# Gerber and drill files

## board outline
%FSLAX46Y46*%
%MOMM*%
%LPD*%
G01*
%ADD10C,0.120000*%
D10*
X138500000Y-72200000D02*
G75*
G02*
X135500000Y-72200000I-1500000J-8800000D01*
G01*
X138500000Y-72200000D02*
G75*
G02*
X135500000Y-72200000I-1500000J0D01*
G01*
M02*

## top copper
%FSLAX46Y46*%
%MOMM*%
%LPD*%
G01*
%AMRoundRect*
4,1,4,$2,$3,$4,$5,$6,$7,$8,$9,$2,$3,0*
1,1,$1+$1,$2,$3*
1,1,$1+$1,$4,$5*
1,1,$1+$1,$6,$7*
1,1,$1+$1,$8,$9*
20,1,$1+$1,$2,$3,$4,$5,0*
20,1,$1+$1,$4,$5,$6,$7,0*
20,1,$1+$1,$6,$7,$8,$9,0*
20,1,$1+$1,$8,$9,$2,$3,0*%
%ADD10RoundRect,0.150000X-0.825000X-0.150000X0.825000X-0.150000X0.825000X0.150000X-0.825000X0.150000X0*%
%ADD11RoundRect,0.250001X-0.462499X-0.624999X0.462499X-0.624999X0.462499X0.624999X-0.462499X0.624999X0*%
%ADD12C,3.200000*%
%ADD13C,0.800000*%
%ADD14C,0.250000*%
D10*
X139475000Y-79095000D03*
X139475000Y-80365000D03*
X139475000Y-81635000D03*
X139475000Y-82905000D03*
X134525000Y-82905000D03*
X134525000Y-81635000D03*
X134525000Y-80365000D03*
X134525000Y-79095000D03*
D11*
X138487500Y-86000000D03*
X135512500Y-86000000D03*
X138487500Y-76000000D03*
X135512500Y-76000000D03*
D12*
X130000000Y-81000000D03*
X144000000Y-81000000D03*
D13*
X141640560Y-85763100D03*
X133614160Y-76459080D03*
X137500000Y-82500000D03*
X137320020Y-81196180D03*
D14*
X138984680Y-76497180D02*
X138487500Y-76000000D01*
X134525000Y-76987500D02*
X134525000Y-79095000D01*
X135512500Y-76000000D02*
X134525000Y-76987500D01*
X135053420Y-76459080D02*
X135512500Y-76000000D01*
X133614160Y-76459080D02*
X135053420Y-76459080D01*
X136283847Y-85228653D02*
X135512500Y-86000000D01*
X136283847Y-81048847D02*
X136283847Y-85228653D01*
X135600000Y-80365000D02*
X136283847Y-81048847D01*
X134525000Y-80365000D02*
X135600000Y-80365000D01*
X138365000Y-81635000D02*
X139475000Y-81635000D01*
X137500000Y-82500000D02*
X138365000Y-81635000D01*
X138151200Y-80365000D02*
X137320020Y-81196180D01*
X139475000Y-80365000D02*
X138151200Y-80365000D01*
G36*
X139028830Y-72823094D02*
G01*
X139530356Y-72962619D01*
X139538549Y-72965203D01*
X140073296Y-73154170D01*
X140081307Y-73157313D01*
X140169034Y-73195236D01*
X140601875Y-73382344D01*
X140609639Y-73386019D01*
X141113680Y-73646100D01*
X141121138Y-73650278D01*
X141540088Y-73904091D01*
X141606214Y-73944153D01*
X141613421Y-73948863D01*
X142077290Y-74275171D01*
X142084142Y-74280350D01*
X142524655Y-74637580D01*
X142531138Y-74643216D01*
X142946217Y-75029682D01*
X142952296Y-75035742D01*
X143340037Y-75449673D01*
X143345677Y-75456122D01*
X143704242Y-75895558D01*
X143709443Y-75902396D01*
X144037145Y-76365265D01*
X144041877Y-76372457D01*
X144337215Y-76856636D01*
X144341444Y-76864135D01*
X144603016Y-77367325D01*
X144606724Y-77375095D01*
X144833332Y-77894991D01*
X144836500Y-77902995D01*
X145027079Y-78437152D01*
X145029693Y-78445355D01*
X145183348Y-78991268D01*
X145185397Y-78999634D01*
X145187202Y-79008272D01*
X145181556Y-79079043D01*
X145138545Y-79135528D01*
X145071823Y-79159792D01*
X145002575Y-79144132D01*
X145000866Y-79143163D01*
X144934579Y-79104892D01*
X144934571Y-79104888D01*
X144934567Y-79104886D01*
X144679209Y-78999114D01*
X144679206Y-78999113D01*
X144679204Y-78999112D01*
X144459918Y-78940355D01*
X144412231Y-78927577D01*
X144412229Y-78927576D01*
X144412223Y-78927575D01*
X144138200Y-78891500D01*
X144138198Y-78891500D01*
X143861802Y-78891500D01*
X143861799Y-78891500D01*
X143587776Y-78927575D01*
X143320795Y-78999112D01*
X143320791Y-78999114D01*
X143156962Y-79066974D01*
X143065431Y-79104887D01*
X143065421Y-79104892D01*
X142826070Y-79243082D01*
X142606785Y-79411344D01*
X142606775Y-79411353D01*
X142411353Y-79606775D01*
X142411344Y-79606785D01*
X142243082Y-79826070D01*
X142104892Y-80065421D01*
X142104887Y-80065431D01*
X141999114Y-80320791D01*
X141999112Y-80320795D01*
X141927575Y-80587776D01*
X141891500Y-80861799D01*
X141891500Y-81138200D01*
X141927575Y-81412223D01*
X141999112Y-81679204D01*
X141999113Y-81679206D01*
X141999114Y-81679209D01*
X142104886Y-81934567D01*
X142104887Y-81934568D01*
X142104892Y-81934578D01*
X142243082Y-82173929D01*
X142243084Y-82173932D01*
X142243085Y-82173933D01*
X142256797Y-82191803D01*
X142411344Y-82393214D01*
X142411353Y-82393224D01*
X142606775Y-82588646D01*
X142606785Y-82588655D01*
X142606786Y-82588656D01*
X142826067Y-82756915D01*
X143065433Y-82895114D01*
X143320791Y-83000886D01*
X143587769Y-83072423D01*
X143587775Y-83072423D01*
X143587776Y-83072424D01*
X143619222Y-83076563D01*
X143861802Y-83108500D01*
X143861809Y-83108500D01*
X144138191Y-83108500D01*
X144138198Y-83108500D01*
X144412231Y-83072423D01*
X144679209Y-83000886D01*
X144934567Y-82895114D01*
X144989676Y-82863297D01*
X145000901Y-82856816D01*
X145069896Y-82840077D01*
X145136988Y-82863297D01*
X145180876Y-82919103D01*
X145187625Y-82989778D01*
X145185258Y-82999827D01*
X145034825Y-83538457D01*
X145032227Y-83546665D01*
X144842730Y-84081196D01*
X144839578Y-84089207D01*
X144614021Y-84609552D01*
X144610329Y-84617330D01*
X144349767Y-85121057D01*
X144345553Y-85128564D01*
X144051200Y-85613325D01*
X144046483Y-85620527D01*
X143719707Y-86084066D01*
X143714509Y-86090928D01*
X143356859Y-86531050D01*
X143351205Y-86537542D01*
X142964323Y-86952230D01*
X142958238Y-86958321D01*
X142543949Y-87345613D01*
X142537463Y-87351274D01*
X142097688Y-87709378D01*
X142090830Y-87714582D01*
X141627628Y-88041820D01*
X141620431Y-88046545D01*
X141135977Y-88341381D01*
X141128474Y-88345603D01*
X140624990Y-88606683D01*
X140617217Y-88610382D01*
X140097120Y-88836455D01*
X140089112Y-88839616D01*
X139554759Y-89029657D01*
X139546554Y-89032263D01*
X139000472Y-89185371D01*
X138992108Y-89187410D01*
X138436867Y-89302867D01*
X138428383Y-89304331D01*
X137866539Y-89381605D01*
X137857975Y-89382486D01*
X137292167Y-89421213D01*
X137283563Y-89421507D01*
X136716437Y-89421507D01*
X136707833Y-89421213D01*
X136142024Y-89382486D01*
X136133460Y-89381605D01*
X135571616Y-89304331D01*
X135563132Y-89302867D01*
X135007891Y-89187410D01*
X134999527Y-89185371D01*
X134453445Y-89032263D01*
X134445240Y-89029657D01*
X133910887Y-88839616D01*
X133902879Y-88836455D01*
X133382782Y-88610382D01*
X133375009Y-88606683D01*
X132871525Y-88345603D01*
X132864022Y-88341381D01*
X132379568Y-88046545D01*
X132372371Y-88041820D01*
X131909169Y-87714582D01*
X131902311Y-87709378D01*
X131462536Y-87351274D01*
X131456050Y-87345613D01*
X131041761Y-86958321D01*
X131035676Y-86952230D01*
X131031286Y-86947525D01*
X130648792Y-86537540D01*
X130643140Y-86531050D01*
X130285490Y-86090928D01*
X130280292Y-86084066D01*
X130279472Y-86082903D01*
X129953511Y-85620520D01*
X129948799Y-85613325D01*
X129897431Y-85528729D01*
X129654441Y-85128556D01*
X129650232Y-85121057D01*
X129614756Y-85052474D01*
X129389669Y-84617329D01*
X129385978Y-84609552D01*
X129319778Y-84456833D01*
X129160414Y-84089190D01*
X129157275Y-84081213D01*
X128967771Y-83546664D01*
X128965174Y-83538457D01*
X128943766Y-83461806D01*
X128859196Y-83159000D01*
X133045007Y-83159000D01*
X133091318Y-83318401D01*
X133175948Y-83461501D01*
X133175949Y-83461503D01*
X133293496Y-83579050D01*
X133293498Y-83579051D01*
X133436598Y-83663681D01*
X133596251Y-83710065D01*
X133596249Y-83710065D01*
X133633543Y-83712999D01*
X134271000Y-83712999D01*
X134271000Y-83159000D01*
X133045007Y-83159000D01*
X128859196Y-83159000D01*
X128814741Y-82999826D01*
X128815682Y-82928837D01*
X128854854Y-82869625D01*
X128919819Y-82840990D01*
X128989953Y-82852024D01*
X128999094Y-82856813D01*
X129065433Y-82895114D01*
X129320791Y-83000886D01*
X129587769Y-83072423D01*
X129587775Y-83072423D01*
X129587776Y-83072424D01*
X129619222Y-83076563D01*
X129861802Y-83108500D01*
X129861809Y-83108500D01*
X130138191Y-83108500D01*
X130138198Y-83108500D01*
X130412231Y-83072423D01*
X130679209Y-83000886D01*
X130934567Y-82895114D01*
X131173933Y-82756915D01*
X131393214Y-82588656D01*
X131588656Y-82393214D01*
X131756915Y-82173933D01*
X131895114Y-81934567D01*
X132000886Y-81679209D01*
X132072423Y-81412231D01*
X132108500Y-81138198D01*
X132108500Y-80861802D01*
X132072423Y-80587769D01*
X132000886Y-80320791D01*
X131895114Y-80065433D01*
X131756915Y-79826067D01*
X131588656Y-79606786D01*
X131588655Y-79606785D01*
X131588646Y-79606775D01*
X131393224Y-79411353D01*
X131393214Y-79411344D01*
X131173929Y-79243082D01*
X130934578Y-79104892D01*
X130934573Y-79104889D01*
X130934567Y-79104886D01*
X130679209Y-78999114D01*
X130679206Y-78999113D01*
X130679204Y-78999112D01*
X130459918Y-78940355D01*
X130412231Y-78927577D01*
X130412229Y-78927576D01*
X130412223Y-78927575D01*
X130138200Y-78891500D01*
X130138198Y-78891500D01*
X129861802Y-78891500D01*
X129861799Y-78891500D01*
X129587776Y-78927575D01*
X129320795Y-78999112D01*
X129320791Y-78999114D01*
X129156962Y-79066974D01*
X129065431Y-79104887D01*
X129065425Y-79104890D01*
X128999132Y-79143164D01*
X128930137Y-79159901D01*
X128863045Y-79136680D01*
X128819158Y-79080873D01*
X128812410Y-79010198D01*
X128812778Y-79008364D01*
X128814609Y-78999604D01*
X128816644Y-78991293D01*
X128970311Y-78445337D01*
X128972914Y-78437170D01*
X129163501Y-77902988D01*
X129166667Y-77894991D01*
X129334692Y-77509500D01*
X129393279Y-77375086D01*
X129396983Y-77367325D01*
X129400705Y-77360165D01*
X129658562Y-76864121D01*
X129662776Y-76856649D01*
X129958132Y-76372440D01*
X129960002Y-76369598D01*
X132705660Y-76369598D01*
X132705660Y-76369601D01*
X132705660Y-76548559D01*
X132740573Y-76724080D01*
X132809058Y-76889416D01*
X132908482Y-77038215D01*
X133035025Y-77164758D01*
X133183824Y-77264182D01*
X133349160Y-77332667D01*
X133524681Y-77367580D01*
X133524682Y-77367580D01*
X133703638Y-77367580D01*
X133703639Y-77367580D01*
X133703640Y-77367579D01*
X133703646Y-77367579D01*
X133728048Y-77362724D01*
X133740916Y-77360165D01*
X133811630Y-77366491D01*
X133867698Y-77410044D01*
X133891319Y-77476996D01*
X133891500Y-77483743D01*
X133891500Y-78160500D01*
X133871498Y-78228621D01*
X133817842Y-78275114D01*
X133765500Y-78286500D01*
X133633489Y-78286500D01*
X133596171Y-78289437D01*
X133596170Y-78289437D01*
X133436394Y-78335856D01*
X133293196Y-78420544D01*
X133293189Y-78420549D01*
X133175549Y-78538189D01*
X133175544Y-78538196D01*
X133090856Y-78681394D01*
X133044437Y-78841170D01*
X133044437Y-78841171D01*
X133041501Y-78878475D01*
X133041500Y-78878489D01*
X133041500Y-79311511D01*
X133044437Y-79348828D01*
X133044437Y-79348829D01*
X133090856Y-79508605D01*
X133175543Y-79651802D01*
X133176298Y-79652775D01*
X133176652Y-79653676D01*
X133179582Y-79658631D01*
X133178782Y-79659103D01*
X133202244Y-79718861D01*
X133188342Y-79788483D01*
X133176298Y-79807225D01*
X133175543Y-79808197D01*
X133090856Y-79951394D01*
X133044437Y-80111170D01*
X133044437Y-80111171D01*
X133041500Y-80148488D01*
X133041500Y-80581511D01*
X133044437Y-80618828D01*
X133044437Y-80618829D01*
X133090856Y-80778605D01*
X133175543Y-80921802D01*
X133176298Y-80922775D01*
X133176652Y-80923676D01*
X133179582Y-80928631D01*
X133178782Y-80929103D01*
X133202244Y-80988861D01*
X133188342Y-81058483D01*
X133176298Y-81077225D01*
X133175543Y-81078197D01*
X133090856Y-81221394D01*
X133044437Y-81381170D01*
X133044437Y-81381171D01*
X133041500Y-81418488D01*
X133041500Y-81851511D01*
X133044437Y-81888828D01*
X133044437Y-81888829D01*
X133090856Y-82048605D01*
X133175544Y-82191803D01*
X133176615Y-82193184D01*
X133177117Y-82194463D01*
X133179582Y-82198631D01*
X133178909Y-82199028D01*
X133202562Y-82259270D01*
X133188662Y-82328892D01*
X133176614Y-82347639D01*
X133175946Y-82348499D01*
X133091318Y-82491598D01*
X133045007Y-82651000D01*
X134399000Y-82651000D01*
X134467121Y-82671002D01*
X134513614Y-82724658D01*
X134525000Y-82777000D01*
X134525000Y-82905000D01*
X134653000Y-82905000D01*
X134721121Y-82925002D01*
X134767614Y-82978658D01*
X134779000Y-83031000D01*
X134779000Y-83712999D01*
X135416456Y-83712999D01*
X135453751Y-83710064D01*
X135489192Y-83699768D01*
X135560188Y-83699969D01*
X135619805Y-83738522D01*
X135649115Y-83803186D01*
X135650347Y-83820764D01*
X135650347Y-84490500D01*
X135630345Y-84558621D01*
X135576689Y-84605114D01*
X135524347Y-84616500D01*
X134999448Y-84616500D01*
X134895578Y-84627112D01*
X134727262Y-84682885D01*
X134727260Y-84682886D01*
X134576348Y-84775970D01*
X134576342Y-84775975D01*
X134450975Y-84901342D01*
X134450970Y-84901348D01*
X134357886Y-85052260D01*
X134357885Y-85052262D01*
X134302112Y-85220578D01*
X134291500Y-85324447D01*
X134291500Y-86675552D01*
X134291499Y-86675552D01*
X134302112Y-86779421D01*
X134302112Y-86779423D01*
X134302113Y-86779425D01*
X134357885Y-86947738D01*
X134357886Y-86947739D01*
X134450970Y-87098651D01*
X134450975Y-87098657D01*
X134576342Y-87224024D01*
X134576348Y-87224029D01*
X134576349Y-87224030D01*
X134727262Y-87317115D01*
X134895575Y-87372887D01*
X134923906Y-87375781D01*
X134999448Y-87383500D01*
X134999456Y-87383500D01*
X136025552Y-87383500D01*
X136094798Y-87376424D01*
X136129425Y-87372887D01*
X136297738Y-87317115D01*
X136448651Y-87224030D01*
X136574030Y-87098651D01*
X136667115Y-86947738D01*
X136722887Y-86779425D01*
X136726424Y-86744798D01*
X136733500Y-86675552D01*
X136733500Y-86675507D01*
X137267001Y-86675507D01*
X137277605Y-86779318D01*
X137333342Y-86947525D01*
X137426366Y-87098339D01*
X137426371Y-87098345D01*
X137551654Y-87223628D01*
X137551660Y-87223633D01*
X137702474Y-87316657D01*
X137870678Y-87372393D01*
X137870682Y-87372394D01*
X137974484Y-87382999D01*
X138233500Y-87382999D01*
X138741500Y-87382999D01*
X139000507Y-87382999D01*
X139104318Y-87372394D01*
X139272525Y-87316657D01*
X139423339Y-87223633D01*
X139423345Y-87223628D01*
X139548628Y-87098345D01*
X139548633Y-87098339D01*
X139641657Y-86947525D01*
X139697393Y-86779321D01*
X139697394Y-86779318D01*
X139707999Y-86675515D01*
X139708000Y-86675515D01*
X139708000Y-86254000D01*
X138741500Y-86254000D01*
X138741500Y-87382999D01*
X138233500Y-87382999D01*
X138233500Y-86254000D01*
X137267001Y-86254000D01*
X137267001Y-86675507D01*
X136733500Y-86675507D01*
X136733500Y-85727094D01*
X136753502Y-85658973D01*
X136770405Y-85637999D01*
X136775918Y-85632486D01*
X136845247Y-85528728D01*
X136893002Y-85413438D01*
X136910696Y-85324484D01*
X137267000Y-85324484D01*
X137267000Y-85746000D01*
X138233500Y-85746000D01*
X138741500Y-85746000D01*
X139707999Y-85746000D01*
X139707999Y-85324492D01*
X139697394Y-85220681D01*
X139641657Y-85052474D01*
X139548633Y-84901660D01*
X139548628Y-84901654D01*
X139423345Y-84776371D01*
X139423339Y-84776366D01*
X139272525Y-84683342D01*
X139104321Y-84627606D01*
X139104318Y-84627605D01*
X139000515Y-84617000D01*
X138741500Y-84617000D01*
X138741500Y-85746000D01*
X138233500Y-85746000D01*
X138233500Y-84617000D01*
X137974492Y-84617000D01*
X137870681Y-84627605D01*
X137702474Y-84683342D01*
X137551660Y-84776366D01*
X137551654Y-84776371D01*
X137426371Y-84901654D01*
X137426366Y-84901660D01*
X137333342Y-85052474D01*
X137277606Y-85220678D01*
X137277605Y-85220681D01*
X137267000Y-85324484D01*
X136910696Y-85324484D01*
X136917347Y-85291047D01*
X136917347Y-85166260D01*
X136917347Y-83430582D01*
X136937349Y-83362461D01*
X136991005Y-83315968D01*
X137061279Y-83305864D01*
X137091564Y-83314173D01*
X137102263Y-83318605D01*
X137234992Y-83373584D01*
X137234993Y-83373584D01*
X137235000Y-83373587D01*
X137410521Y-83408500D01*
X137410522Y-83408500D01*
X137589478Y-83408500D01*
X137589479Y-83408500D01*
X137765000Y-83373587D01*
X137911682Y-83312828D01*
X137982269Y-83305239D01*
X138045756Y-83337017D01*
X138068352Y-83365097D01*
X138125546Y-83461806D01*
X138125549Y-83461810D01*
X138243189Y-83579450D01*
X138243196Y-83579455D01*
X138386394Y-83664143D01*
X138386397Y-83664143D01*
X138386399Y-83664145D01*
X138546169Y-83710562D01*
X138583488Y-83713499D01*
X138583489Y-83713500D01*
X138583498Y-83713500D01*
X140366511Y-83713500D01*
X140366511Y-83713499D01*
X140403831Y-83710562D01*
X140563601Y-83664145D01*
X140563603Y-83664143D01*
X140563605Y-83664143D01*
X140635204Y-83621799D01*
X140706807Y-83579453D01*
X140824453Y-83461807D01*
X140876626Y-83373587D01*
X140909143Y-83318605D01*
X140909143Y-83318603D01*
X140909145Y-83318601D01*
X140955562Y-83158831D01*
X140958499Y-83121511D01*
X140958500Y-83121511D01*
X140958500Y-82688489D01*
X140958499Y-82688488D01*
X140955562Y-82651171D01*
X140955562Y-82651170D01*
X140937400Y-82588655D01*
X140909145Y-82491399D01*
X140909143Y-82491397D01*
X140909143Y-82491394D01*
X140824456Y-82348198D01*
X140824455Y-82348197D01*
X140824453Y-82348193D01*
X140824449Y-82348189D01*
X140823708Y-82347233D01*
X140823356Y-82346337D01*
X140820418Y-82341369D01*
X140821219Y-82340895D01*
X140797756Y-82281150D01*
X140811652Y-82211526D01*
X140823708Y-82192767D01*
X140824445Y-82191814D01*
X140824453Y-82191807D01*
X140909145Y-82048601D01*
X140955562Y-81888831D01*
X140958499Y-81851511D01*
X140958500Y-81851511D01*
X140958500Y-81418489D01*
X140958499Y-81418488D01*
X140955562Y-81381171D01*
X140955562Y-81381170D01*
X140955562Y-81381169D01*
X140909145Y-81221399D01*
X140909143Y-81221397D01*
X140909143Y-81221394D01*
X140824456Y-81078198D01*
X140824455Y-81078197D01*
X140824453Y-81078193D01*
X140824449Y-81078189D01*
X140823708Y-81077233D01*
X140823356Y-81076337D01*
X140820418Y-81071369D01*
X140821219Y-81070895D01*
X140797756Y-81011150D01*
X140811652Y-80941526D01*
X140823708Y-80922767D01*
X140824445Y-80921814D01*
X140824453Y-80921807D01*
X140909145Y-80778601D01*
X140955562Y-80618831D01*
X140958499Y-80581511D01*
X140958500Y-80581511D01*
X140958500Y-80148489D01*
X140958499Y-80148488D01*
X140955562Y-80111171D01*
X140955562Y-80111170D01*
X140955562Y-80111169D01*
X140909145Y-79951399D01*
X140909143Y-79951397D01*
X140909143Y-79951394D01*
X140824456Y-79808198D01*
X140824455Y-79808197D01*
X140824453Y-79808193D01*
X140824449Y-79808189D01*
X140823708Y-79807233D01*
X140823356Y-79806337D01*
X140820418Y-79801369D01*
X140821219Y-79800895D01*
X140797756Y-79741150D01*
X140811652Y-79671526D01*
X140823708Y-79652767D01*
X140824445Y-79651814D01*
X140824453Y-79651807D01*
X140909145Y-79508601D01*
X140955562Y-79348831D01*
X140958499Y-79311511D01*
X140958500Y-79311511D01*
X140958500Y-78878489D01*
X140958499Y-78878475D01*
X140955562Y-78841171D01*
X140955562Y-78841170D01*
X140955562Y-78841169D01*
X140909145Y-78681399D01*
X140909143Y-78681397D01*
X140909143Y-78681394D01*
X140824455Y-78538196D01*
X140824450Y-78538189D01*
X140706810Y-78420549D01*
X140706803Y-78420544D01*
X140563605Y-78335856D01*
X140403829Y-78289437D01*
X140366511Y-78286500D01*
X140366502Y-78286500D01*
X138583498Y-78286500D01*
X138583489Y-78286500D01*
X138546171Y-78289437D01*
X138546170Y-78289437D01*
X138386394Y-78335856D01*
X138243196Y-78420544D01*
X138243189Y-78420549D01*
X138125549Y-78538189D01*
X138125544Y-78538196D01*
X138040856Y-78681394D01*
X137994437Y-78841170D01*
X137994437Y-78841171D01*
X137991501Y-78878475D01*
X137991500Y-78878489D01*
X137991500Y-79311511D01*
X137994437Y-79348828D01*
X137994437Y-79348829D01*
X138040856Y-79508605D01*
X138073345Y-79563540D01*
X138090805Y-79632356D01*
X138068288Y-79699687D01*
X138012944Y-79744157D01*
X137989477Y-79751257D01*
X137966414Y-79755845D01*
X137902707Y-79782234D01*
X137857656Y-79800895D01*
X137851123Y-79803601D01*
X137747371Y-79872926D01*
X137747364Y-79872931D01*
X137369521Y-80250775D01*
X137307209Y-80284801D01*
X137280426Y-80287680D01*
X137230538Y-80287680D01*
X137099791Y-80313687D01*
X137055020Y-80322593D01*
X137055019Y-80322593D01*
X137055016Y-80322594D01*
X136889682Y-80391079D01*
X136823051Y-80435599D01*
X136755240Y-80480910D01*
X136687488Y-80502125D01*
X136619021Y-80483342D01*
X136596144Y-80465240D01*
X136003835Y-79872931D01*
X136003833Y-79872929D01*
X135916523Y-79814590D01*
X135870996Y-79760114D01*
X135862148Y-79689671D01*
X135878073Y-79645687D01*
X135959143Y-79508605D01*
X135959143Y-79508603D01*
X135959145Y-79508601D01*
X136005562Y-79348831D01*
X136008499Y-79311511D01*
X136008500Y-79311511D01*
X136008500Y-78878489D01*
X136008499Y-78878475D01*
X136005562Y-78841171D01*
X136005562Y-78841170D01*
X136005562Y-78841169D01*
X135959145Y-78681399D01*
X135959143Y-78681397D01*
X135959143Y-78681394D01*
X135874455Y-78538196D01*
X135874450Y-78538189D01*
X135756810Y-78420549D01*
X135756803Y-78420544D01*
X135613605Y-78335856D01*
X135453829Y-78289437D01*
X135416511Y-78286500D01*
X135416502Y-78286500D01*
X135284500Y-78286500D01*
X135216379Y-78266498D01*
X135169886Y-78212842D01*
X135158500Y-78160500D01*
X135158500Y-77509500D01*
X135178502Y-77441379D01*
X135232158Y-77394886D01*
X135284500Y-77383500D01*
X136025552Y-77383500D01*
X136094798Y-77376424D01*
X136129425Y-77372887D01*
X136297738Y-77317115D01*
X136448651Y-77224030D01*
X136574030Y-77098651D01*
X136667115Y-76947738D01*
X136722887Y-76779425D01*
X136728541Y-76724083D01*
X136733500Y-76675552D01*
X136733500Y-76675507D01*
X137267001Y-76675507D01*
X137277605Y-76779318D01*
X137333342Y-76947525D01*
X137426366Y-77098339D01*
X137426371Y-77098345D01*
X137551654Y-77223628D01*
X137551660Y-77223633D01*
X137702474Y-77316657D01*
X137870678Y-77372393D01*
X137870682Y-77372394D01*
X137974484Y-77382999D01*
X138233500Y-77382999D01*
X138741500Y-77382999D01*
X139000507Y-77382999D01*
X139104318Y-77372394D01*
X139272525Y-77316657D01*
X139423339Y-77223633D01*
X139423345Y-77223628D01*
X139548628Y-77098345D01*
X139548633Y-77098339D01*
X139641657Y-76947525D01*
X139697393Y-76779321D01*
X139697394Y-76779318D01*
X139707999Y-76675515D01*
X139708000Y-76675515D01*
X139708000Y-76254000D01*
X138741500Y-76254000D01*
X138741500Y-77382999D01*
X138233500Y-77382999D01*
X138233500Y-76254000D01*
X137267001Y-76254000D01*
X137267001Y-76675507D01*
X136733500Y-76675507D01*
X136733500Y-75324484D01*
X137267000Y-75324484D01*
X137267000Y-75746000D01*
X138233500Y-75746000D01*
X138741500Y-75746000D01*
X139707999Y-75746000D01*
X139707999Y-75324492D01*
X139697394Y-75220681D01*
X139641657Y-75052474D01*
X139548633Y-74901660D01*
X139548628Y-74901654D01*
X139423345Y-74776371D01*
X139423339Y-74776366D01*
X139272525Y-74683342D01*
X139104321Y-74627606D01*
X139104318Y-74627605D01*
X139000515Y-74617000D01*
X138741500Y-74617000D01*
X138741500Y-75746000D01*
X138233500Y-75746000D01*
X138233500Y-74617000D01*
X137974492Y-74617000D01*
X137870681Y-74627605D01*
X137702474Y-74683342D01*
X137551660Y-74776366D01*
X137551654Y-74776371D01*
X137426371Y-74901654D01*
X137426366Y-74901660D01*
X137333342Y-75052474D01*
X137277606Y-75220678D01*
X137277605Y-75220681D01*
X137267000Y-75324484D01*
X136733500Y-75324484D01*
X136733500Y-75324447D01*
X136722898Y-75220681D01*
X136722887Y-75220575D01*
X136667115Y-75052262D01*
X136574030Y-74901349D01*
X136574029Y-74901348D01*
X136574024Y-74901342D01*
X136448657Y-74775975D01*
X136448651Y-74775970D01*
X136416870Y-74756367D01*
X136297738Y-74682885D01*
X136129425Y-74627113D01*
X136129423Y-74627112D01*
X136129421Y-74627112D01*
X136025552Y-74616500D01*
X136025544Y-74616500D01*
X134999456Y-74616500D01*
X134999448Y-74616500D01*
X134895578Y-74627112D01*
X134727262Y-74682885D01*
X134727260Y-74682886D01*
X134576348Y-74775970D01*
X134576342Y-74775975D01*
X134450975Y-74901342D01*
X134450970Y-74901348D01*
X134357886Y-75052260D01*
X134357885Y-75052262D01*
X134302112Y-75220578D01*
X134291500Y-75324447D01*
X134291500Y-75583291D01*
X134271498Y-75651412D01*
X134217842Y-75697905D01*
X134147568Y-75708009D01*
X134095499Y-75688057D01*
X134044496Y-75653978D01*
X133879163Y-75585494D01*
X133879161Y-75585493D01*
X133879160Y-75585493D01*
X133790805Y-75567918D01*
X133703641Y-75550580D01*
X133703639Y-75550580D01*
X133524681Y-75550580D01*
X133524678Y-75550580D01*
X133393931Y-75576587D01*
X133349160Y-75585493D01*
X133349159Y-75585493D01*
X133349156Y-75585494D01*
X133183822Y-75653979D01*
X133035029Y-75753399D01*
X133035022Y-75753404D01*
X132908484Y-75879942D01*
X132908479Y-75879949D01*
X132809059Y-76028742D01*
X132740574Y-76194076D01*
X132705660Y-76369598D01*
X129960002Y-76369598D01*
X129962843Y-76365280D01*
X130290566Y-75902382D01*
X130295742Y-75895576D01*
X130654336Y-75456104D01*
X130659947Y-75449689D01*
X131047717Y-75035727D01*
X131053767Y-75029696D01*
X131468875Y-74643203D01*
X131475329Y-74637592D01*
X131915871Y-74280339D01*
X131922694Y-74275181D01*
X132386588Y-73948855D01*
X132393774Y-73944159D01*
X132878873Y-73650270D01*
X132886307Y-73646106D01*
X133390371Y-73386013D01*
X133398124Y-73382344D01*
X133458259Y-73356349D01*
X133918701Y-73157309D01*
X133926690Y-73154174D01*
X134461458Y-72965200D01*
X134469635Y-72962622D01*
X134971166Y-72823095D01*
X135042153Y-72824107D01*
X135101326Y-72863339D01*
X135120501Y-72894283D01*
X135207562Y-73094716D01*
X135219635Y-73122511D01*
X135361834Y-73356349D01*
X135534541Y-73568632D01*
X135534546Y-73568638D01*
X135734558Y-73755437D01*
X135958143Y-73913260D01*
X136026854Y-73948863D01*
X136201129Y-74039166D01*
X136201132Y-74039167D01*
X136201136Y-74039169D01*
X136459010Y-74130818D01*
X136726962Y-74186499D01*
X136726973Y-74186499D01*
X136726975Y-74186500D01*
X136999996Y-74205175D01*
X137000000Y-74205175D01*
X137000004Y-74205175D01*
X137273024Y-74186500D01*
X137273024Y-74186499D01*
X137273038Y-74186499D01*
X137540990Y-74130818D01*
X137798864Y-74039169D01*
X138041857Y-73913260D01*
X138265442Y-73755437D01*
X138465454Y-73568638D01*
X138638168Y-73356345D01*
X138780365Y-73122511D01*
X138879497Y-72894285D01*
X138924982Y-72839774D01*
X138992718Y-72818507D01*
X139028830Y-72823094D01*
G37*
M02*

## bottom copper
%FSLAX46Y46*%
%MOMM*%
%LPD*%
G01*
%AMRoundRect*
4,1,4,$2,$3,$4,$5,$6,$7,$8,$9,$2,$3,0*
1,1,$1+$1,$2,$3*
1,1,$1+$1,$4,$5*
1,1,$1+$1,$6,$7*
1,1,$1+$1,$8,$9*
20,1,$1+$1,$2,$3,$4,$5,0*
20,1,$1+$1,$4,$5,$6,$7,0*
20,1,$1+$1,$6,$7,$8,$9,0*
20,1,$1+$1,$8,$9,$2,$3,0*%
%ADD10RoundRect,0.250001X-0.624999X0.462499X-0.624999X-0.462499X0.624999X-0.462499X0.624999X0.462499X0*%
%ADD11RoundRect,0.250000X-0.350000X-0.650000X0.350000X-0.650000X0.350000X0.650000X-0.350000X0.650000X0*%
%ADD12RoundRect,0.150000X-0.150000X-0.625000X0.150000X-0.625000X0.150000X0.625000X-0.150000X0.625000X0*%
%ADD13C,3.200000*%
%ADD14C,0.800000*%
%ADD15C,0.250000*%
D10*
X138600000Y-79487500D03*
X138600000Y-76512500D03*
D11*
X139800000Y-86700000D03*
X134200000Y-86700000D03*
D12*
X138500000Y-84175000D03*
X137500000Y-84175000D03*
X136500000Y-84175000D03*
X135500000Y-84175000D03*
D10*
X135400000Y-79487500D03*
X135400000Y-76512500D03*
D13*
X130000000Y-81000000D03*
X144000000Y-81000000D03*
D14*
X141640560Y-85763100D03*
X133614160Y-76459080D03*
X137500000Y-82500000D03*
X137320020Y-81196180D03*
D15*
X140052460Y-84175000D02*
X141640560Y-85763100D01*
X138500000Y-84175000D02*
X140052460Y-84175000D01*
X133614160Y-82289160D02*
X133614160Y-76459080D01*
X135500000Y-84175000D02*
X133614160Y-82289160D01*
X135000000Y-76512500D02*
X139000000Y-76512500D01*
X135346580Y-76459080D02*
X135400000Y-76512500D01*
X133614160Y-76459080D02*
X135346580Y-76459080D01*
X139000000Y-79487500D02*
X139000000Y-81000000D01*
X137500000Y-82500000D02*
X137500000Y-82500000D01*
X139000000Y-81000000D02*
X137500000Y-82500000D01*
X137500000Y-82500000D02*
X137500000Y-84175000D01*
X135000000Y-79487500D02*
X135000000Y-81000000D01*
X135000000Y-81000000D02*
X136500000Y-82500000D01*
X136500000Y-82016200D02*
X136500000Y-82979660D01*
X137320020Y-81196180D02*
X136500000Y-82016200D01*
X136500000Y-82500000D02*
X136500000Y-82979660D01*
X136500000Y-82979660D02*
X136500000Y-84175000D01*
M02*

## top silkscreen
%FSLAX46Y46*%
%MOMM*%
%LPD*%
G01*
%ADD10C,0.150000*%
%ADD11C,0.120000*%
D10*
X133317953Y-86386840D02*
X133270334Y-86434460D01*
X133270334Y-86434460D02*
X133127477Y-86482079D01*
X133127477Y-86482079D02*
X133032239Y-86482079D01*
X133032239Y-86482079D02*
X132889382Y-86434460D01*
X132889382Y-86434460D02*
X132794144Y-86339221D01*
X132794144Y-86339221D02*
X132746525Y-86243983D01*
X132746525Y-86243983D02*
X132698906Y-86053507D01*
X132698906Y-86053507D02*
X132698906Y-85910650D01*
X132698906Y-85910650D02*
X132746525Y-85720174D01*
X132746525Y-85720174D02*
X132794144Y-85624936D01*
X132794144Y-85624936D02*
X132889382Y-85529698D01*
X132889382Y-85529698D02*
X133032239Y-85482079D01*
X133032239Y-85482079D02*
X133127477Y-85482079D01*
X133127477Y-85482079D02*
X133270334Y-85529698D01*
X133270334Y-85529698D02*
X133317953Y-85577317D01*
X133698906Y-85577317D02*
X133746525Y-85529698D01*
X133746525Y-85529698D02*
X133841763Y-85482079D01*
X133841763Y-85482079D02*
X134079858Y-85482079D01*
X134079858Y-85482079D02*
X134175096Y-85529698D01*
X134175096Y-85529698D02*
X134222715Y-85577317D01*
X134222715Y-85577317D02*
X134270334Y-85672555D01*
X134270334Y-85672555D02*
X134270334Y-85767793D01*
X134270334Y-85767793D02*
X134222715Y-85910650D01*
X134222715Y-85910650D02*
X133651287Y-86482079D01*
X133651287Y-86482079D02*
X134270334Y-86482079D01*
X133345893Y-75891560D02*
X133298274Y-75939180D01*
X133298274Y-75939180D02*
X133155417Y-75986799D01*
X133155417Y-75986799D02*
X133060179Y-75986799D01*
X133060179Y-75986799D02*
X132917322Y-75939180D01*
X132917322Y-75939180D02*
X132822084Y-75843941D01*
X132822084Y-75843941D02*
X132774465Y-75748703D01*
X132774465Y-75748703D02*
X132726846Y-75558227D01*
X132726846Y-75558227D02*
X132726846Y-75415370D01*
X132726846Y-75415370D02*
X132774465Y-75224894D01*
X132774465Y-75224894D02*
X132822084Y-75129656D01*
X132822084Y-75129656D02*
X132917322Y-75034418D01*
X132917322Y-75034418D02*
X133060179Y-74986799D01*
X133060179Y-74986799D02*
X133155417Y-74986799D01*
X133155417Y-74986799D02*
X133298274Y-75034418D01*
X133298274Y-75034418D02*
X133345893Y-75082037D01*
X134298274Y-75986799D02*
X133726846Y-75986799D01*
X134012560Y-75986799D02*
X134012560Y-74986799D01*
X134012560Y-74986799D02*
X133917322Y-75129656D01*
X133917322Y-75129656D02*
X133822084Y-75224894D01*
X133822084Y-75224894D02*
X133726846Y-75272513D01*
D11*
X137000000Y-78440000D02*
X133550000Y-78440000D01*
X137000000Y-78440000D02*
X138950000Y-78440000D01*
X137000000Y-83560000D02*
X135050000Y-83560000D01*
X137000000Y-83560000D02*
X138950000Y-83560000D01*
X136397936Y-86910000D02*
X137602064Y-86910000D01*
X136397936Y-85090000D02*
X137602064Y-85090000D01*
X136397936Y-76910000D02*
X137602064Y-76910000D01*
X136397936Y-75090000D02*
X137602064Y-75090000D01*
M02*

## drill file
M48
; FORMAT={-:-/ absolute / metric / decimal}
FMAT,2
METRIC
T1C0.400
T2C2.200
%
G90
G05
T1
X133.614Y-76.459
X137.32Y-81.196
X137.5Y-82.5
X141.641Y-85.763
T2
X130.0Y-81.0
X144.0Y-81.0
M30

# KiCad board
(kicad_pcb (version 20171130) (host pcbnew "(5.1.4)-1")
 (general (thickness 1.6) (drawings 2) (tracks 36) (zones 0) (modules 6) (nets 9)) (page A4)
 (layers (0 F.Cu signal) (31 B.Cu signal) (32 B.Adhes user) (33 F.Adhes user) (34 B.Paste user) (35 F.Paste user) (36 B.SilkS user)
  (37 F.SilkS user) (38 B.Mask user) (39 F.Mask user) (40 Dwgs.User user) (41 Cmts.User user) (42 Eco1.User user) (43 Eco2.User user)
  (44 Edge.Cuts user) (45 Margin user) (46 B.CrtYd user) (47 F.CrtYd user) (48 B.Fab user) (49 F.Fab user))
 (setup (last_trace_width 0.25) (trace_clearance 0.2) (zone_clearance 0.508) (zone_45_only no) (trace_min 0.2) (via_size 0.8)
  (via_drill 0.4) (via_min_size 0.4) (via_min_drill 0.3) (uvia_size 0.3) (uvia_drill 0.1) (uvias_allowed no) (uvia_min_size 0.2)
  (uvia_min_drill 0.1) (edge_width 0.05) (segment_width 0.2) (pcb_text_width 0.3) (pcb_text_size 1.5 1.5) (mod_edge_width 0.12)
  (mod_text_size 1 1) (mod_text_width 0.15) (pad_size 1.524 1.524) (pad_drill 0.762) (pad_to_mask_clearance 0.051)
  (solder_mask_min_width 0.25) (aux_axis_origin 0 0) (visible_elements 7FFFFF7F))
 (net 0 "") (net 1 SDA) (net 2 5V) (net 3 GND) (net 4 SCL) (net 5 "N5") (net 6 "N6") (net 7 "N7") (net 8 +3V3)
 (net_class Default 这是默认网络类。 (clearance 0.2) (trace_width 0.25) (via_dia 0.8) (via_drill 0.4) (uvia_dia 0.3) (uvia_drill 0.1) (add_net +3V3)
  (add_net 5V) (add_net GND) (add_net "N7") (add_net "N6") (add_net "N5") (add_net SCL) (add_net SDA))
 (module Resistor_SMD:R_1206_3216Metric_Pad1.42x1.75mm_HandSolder (layer B.Cu) (at 138.6 78 270)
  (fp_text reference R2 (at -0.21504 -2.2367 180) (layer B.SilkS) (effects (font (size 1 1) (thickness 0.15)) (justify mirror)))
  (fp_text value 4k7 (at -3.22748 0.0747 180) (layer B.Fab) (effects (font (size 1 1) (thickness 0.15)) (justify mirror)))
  (pad 2 smd roundrect (at 1.4875 0 270) (size 1.425 1.75) (layers B.Cu B.Paste B.Mask) (roundrect_rratio 0.175439) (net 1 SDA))
  (pad 1 smd roundrect (at -1.4875 0 270) (size 1.425 1.75) (layers B.Cu B.Paste B.Mask) (roundrect_rratio 0.175439) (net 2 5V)))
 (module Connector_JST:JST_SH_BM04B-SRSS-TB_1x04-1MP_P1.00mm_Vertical (layer B.Cu) (at 137 85.5)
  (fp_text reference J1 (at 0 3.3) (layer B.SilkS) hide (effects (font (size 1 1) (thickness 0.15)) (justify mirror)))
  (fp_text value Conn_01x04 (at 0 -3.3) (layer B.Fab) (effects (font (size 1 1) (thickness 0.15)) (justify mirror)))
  (pad MP smd roundrect (at 2.8 1.2) (size 1.2 1.8) (layers B.Cu B.Paste B.Mask) (roundrect_rratio 0.208333))
  (pad MP smd roundrect (at -2.8 1.2) (size 1.2 1.8) (layers B.Cu B.Paste B.Mask) (roundrect_rratio 0.208333))
  (pad 4 smd roundrect (at 1.5 -1.325) (size 0.6 1.55) (layers B.Cu B.Paste B.Mask) (roundrect_rratio 0.25) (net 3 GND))
  (pad 3 smd roundrect (at 0.5 -1.325) (size 0.6 1.55) (layers B.Cu B.Paste B.Mask) (roundrect_rratio 0.25) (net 1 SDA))
  (pad 2 smd roundrect (at -0.5 -1.325) (size 0.6 1.55) (layers B.Cu B.Paste B.Mask) (roundrect_rratio 0.25) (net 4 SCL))
  (pad 1 smd roundrect (at -1.5 -1.325) (size 0.6 1.55) (layers B.Cu B.Paste B.Mask) (roundrect_rratio 0.25) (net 2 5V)))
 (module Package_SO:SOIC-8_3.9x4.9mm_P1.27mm (layer F.Cu) (at 137 81)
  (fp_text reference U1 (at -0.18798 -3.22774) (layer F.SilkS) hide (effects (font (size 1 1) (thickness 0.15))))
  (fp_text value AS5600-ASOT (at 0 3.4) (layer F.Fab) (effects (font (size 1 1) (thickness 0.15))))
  (fp_line (start 0 -2.56) (end -3.45 -2.56) (layer F.SilkS) (width 0.12))
  (fp_line (start 0 -2.56) (end 1.95 -2.56) (layer F.SilkS) (width 0.12))
  (fp_line (start 0 2.56) (end -1.95 2.56) (layer F.SilkS) (width 0.12))
  (fp_line (start 0 2.56) (end 1.95 2.56) (layer F.SilkS) (width 0.12))
  (pad 8 smd roundrect (at 2.475 -1.905) (size 1.95 0.6) (layers F.Cu F.Paste F.Mask) (roundrect_rratio 0.25) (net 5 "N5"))
  (pad 7 smd roundrect (at 2.475 -0.635) (size 1.95 0.6) (layers F.Cu F.Paste F.Mask) (roundrect_rratio 0.25) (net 4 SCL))
  (pad 6 smd roundrect (at 2.475 0.635) (size 1.95 0.6) (layers F.Cu F.Paste F.Mask) (roundrect_rratio 0.25) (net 1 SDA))
  (pad 5 smd roundrect (at 2.475 1.905) (size 1.95 0.6) (layers F.Cu F.Paste F.Mask) (roundrect_rratio 0.25) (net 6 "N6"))
  (pad 4 smd roundrect (at -2.475 1.905) (size 1.95 0.6) (layers F.Cu F.Paste F.Mask) (roundrect_rratio 0.25) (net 3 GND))
  (pad 3 smd roundrect (at -2.475 0.635) (size 1.95 0.6) (layers F.Cu F.Paste F.Mask) (roundrect_rratio 0.25) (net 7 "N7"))
  (pad 2 smd roundrect (at -2.475 -0.635) (size 1.95 0.6) (layers F.Cu F.Paste F.Mask) (roundrect_rratio 0.25) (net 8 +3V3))
  (pad 1 smd roundrect (at -2.475 -1.905) (size 1.95 0.6) (layers F.Cu F.Paste F.Mask) (roundrect_rratio 0.25) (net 2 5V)))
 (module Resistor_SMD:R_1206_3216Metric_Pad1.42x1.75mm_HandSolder (layer B.Cu) (at 135.4 78 270)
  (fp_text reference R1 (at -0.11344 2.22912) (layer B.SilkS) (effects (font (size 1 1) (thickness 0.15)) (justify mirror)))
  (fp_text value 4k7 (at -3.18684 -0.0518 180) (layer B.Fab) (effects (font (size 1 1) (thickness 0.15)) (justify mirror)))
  (pad 2 smd roundrect (at 1.4875 0 270) (size 1.425 1.75) (layers B.Cu B.Paste B.Mask) (roundrect_rratio 0.175439) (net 4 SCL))
  (pad 1 smd roundrect (at -1.4875 0 270) (size 1.425 1.75) (layers B.Cu B.Paste B.Mask) (roundrect_rratio 0.175439) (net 2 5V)))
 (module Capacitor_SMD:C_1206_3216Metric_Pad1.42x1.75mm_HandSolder (layer F.Cu) (at 137 86)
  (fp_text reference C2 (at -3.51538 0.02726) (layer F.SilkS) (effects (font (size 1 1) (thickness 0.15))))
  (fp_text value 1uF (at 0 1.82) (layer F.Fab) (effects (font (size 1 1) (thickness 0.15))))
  (fp_line (start -0.602064 0.91) (end 0.602064 0.91) (layer F.SilkS) (width 0.12))
  (fp_line (start -0.602064 -0.91) (end 0.602064 -0.91) (layer F.SilkS) (width 0.12))
  (pad 2 smd roundrect (at 1.4875 0) (size 1.425 1.75) (layers F.Cu F.Paste F.Mask) (roundrect_rratio 0.175439) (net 3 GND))
  (pad 1 smd roundrect (at -1.4875 0) (size 1.425 1.75) (layers F.Cu F.Paste F.Mask) (roundrect_rratio 0.175439) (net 8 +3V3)))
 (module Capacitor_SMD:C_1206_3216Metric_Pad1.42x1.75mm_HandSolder (layer F.Cu) (at 137 76)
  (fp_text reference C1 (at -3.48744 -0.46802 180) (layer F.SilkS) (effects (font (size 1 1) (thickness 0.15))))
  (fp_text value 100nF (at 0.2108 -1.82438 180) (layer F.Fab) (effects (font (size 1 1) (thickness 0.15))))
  (fp_line (start -0.602064 0.91) (end 0.602064 0.91) (layer F.SilkS) (width 0.12))
  (fp_line (start -0.602064 -0.91) (end 0.602064 -0.91) (layer F.SilkS) (width 0.12))
  (pad 2 smd roundrect (at 1.4875 0) (size 1.425 1.75) (layers F.Cu F.Paste F.Mask) (roundrect_rratio 0.175439) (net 3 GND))
  (pad 1 smd roundrect (at -1.4875 0) (size 1.425 1.75) (layers F.Cu F.Paste F.Mask) (roundrect_rratio 0.175439) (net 2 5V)))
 (gr_arc (start 137 81) (end 135.5 72.2) (angle -340.6532891) (layer Edge.Cuts) (width 0.12))
 (gr_arc (start 137 72.2) (end 135.5 72.2) (angle -180) (layer Edge.Cuts) (width 0.12))
 (via (at 130 81) (size 3.2) (drill 2.2) (layers F.Cu B.Cu) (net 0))
 (via (at 144 81) (size 3.2) (drill 2.2) (layers F.Cu B.Cu) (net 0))
 (via (at 141.64056 85.7631) (size 0.8) (drill 0.4) (layers F.Cu B.Cu) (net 3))
 (segment (start 138.98468 76.49718) (end 138.4875 76) (width 0.25) (layer F.Cu) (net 3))
 (segment (start 140.05246 84.175) (end 141.64056 85.7631) (width 0.25) (layer B.Cu) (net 3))
 (segment (start 138.5 84.175) (end 140.05246 84.175) (width 0.25) (layer B.Cu) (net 3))
 (via (at 133.61416 76.45908) (size 0.8) (drill 0.4) (layers F.Cu B.Cu) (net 2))
 (segment (start 133.61416 82.28916) (end 133.61416 76.45908) (width 0.25) (layer B.Cu) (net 2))
 (segment (start 135.5 84.175) (end 133.61416 82.28916) (width 0.25) (layer B.Cu) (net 2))
 (segment (start 135 76.5125) (end 139 76.5125) (width 0.25) (layer B.Cu) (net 2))
 (segment (start 134.525 76.9875) (end 134.525 79.095) (width 0.25) (layer F.Cu) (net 2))
 (segment (start 135.5125 76) (end 134.525 76.9875) (width 0.25) (layer F.Cu) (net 2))
 (segment (start 135.34658 76.45908) (end 135.4 76.5125) (width 0.25) (layer B.Cu) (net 2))
 (segment (start 133.61416 76.45908) (end 135.34658 76.45908) (width 0.25) (layer B.Cu) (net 2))
 (segment (start 135.05342 76.45908) (end 135.5125 76) (width 0.25) (layer F.Cu) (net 2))
 (segment (start 133.61416 76.45908) (end 135.05342 76.45908) (width 0.25) (layer F.Cu) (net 2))
 (segment (start 136.283847 85.228653) (end 135.5125 86) (width 0.25) (layer F.Cu) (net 8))
 (segment (start 136.283847 81.048847) (end 136.283847 85.228653) (width 0.25) (layer F.Cu) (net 8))
 (segment (start 135.6 80.365) (end 136.283847 81.048847) (width 0.25) (layer F.Cu) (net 8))
 (segment (start 134.525 80.365) (end 135.6 80.365) (width 0.25) (layer F.Cu) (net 8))
 (segment (start 139 79.4875) (end 139 81) (width 0.25) (layer B.Cu) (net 1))
 (segment (start 137.5 82.5) (end 137.5 82.5) (width 0.25) (layer B.Cu) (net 1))
 (segment (start 139 81) (end 137.5 82.5) (width 0.25) (layer B.Cu) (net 1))
 (segment (start 137.5 82.5) (end 137.5 84.175) (width 0.25) (layer B.Cu) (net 1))
 (via (at 137.5 82.5) (size 0.8) (drill 0.4) (layers F.Cu B.Cu) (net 1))
 (segment (start 138.365 81.635) (end 139.475 81.635) (width 0.25) (layer F.Cu) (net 1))
 (segment (start 137.5 82.5) (end 138.365 81.635) (width 0.25) (layer F.Cu) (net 1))
 (via (at 137.32002 81.19618) (size 0.8) (drill 0.4) (layers F.Cu B.Cu) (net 4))
 (segment (start 135 79.4875) (end 135 81) (width 0.25) (layer B.Cu) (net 4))
 (segment (start 135 81) (end 136.5 82.5) (width 0.25) (layer B.Cu) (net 4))
 (segment (start 138.1512 80.365) (end 137.32002 81.19618) (width 0.25) (layer F.Cu) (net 4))
 (segment (start 139.475 80.365) (end 138.1512 80.365) (width 0.25) (layer F.Cu) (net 4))
 (segment (start 136.5 82.0162) (end 136.5 82.97966) (width 0.25) (layer B.Cu) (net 4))
 (segment (start 137.32002 81.19618) (end 136.5 82.0162) (width 0.25) (layer B.Cu) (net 4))
 (segment (start 136.5 82.5) (end 136.5 82.97966) (width 0.25) (layer B.Cu) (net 4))
 (segment (start 136.5 82.97966) (end 136.5 84.175) (width 0.25) (layer B.Cu) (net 4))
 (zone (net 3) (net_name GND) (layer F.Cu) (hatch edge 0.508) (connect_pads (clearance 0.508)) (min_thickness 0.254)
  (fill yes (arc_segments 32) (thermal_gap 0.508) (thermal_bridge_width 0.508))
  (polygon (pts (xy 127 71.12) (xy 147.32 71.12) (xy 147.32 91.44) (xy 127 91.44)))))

